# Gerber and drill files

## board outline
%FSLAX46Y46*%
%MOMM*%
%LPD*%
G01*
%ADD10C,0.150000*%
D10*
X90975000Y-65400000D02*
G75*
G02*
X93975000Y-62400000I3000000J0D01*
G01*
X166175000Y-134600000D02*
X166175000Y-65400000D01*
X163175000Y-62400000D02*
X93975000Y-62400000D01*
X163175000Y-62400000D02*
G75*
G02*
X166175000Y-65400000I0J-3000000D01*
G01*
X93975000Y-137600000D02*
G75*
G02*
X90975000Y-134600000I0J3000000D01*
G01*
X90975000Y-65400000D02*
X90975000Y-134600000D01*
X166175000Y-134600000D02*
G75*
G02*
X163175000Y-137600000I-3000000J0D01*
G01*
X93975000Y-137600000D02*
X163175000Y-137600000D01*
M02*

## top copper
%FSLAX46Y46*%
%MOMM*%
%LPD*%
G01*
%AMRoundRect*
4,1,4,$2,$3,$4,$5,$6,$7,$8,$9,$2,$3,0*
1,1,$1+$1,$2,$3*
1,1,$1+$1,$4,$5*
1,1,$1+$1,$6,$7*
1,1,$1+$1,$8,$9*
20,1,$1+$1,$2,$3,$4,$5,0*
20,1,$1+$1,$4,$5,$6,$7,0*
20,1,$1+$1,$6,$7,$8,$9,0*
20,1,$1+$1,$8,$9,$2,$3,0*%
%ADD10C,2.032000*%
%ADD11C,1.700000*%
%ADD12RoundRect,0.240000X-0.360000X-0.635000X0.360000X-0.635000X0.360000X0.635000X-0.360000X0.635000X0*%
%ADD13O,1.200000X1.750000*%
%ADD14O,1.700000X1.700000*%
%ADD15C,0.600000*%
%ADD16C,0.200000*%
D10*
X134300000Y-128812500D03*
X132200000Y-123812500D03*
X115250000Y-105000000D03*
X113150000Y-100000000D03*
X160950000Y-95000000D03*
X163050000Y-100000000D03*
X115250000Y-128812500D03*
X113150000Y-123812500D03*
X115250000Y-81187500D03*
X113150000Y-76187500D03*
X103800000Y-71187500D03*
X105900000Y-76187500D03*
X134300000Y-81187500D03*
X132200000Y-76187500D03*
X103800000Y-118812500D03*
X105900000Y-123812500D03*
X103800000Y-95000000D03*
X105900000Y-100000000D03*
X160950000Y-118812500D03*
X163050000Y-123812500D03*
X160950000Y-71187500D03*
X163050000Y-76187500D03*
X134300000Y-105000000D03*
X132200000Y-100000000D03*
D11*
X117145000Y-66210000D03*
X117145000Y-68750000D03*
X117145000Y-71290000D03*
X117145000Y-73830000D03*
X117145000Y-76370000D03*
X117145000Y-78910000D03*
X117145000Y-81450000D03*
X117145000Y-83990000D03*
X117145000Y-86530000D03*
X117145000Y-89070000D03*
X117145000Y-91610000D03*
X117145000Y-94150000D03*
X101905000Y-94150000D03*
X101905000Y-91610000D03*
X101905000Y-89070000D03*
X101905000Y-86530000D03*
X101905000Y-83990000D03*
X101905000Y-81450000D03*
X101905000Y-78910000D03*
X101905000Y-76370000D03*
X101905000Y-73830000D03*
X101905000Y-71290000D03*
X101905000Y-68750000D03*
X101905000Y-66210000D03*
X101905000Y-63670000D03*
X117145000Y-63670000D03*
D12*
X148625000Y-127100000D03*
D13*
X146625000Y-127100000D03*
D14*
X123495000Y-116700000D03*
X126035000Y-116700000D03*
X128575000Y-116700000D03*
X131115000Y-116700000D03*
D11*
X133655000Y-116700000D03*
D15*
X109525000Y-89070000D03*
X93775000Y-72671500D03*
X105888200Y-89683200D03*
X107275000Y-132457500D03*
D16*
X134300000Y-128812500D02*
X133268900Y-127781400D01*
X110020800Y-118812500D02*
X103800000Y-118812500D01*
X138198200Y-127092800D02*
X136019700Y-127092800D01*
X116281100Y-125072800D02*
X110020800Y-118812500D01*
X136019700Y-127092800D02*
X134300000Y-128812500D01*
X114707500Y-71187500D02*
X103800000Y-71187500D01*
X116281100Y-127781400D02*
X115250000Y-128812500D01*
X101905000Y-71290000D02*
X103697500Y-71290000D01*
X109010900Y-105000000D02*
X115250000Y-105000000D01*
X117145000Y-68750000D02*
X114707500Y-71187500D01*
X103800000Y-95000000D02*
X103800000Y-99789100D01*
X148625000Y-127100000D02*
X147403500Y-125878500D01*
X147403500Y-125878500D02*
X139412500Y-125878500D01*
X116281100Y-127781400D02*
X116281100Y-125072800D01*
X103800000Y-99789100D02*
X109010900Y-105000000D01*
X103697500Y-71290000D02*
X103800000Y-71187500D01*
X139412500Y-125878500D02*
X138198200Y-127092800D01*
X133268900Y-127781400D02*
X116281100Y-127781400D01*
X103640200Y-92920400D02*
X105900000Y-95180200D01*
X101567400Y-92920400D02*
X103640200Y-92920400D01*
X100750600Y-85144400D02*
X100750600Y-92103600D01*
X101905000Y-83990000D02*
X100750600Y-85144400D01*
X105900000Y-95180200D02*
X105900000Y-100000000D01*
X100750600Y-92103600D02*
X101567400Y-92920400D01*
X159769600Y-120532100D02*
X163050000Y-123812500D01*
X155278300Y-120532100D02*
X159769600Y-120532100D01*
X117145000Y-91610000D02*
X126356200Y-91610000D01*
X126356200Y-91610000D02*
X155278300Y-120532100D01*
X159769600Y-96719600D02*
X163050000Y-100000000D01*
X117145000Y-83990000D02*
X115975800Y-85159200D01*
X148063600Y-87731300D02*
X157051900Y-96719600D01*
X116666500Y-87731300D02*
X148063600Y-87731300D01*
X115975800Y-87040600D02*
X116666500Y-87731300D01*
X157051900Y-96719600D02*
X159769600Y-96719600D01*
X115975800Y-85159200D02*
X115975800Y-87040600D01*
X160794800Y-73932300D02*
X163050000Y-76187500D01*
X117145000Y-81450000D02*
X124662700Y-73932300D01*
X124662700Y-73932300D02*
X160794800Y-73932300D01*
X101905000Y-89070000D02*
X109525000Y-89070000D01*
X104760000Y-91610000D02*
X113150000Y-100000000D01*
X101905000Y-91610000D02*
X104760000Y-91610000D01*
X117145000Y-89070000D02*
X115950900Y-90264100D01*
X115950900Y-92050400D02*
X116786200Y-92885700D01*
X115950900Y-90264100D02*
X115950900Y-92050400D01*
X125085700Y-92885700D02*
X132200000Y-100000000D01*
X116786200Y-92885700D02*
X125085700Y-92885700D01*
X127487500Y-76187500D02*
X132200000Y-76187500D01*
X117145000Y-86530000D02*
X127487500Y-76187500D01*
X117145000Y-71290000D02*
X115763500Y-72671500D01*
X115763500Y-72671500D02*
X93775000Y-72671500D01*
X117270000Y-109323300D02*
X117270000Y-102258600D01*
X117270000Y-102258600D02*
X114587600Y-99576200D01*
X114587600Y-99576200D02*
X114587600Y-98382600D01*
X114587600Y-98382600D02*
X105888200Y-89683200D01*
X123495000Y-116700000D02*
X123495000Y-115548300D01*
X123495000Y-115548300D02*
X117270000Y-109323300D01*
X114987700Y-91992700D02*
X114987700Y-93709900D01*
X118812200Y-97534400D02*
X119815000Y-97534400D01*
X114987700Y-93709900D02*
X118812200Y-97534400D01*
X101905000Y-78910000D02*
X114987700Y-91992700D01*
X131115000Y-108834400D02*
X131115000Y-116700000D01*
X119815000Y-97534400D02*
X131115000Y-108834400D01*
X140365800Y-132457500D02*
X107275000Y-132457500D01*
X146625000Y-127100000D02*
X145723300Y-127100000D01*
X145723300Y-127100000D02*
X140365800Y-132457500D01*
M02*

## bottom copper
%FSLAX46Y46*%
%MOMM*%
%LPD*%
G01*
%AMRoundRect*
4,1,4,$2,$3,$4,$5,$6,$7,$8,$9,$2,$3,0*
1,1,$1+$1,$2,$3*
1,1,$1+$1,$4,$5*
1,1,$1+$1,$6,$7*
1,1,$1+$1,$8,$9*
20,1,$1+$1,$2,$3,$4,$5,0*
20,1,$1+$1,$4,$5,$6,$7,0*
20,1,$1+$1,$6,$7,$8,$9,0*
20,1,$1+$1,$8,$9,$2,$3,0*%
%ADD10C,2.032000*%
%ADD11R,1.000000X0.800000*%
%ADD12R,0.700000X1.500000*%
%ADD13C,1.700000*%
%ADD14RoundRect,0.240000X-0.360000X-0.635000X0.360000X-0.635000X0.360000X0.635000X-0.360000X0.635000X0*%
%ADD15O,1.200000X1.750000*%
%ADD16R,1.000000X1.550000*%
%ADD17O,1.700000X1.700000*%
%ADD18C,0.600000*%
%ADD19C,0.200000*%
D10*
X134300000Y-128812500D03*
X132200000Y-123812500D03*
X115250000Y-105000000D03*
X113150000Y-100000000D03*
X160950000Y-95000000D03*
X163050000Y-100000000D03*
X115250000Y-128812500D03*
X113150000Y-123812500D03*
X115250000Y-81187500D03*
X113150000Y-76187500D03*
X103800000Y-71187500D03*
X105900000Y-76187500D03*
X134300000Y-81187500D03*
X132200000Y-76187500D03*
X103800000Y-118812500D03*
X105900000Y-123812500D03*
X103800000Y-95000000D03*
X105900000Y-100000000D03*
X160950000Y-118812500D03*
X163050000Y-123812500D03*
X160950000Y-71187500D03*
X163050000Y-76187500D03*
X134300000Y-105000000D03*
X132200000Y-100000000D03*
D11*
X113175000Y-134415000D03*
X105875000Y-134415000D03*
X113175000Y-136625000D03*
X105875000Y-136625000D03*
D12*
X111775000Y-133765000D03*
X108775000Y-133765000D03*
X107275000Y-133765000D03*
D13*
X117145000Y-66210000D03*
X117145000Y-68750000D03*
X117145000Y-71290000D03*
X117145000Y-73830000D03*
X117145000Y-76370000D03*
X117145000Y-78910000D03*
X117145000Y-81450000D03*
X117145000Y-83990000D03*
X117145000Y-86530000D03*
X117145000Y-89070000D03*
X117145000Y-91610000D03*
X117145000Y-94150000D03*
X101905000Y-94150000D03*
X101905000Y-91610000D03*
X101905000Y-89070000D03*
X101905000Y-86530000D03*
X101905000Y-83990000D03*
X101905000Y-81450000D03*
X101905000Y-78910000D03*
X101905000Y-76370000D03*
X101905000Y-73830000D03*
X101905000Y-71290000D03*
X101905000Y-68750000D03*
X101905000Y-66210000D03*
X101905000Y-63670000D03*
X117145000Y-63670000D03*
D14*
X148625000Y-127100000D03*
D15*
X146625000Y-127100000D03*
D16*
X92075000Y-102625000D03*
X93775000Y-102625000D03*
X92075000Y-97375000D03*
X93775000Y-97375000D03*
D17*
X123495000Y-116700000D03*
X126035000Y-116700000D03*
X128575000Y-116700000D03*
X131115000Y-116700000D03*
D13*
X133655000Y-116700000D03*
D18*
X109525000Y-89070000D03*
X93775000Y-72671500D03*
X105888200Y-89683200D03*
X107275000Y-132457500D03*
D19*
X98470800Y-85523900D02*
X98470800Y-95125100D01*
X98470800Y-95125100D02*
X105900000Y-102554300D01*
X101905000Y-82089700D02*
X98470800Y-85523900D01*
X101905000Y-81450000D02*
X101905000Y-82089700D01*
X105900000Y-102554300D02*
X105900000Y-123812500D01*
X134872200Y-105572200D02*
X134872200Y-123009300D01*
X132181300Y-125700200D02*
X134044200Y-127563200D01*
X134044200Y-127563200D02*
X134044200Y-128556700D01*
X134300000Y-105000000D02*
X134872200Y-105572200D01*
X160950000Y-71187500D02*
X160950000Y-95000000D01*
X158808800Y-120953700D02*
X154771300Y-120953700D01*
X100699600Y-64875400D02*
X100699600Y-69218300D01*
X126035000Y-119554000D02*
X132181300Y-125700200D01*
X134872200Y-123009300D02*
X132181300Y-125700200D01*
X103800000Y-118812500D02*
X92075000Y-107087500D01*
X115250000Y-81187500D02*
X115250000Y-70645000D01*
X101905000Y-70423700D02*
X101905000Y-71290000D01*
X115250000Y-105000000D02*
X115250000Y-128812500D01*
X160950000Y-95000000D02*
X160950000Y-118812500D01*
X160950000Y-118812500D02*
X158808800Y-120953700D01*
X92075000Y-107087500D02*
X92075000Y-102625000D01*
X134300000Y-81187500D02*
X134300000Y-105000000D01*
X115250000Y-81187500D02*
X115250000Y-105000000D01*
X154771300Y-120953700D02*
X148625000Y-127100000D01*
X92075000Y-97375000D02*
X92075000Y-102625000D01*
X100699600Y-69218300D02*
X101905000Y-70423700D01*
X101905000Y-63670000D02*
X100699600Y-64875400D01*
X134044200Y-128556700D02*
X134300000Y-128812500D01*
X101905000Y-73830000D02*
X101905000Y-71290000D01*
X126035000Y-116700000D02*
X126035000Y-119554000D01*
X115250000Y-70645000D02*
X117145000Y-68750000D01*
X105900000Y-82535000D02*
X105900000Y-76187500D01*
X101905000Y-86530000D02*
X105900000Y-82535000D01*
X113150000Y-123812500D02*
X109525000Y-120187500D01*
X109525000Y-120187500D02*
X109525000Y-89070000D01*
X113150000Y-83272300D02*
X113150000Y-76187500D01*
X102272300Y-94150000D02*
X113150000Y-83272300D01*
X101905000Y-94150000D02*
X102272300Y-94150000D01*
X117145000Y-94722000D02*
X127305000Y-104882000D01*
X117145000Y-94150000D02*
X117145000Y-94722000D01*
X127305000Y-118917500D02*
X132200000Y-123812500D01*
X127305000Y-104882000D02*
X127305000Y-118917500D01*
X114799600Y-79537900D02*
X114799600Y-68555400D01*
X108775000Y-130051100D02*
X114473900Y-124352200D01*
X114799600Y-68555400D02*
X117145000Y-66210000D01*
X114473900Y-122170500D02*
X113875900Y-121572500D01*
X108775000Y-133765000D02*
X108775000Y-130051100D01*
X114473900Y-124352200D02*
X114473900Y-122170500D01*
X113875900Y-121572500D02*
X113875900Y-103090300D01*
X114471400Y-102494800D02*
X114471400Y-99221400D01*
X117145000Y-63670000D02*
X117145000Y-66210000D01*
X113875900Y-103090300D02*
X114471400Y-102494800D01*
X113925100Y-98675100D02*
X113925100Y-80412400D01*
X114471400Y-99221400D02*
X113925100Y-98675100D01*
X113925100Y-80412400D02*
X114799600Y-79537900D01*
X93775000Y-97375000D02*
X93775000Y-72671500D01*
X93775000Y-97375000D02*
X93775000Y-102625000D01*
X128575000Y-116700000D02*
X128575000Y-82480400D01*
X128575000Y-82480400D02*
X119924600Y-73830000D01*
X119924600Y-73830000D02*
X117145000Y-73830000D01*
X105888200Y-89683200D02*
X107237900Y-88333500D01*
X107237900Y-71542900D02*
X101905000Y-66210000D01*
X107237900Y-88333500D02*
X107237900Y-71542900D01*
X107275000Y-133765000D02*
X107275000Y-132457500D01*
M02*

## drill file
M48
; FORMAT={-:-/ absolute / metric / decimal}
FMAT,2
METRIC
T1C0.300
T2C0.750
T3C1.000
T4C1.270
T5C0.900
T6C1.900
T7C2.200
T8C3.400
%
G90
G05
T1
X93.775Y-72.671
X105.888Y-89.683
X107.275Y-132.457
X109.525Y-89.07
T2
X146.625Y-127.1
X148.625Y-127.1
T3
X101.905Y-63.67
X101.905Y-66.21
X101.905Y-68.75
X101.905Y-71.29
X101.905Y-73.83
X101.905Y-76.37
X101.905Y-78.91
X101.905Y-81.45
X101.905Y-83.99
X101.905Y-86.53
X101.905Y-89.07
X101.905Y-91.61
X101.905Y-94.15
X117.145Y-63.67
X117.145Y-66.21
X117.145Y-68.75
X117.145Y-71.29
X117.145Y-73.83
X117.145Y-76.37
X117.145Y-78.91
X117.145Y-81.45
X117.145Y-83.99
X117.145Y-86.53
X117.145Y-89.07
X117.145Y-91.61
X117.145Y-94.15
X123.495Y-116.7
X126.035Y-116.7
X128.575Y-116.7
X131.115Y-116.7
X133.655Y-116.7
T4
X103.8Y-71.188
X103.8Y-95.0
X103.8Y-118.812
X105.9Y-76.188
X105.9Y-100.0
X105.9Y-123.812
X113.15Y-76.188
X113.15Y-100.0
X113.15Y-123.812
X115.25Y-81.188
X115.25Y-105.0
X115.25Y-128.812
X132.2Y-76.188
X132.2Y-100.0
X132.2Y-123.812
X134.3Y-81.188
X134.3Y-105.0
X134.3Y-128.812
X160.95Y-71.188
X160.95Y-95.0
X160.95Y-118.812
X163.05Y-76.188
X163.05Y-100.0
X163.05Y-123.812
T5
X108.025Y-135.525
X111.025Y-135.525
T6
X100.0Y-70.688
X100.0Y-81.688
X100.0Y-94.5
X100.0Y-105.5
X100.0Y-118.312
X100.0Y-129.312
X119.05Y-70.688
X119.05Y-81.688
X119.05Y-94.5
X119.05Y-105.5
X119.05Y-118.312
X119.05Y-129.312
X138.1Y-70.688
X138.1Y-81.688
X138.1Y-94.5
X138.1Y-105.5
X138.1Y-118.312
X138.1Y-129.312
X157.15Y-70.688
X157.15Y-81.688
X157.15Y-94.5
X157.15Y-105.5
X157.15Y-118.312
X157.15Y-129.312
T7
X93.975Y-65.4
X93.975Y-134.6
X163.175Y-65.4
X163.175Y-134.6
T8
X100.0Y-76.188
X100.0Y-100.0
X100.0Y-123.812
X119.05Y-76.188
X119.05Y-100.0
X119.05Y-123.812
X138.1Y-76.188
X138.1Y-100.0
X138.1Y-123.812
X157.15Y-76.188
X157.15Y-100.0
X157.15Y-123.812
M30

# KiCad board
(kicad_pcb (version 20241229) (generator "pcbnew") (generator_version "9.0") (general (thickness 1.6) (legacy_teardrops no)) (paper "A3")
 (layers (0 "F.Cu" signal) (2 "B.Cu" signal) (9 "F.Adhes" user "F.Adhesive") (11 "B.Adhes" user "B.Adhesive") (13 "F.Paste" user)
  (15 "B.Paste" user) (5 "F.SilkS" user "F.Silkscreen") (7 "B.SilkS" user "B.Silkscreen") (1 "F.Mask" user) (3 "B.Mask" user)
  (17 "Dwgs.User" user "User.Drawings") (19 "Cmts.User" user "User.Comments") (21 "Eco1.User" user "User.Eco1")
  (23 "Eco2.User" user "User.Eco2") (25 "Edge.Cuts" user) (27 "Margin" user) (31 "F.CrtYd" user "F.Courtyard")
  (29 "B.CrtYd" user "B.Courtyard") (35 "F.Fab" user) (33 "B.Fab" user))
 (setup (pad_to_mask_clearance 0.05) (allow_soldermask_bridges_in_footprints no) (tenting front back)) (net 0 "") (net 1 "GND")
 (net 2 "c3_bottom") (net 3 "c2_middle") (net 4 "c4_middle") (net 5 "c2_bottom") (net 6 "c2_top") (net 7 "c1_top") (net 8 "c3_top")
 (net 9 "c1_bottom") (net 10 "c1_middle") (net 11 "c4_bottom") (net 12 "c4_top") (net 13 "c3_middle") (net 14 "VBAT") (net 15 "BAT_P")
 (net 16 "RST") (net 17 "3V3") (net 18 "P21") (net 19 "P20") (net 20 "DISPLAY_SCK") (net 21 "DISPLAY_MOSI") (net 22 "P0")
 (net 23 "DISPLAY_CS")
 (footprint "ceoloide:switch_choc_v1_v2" (layer "F.Cu") (at 138.1 123.8125 90)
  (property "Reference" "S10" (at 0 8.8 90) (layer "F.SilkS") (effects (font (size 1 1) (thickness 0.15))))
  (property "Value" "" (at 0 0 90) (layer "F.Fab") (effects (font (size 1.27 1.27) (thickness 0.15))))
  (pad "" np_thru_hole circle (at -5.5 0 90) (size 1.9 1.9) (drill 1.9) (layers "*.Cu" "*.Mask"))
  (pad "" np_thru_hole circle (at 0 0 90) (size 3.4 3.4) (drill 3.4) (layers "*.Cu" "*.Mask"))
  (pad "" np_thru_hole circle (at 5.5 0 90) (size 1.9 1.9) (drill 1.9) (layers "*.Cu" "*.Mask"))
  (pad "1" thru_hole circle (at -5 -3.8 285) (size 2.032 2.032) (drill 1.27) (layers "*.Cu" "*.Mask") (remove_unused_layers no)
   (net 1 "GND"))
  (pad "2" thru_hole circle (at 0 -5.9 285) (size 2.032 2.032) (drill 1.27) (layers "*.Cu" "*.Mask") (remove_unused_layers no)
   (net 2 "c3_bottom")))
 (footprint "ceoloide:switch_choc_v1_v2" (layer "F.Cu") (at 119.05 100 90)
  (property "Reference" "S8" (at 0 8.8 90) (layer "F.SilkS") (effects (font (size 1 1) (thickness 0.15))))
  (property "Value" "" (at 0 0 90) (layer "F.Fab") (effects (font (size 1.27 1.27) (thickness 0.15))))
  (pad "" np_thru_hole circle (at -5.5 0 90) (size 1.9 1.9) (drill 1.9) (layers "*.Cu" "*.Mask"))
  (pad "" np_thru_hole circle (at 0 0 90) (size 3.4 3.4) (drill 3.4) (layers "*.Cu" "*.Mask"))
  (pad "" np_thru_hole circle (at 5.5 0 90) (size 1.9 1.9) (drill 1.9) (layers "*.Cu" "*.Mask"))
  (pad "1" thru_hole circle (at -5 -3.8 285) (size 2.032 2.032) (drill 1.27) (layers "*.Cu" "*.Mask") (remove_unused_layers no)
   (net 1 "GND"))
  (pad "2" thru_hole circle (at 0 -5.9 285) (size 2.032 2.032) (drill 1.27) (layers "*.Cu" "*.Mask") (remove_unused_layers no)
   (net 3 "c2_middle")))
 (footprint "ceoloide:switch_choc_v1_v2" (layer "F.Cu") (at 157.15 100 -90)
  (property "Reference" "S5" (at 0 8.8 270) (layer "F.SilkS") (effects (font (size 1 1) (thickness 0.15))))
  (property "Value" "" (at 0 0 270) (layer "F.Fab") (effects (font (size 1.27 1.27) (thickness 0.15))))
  (pad "" np_thru_hole circle (at -5.5 0 270) (size 1.9 1.9) (drill 1.9) (layers "*.Cu" "*.Mask"))
  (pad "" np_thru_hole circle (at 0 0 270) (size 3.4 3.4) (drill 3.4) (layers "*.Cu" "*.Mask"))
  (pad "" np_thru_hole circle (at 5.5 0 270) (size 1.9 1.9) (drill 1.9) (layers "*.Cu" "*.Mask"))
  (pad "1" thru_hole circle (at -5 -3.8 105) (size 2.032 2.032) (drill 1.27) (layers "*.Cu" "*.Mask") (remove_unused_layers no)
   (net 1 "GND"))
  (pad "2" thru_hole circle (at 0 -5.9 105) (size 2.032 2.032) (drill 1.27) (layers "*.Cu" "*.Mask") (remove_unused_layers no)
   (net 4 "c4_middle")))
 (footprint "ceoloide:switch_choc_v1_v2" (layer "F.Cu") (at 119.05 123.8125 90)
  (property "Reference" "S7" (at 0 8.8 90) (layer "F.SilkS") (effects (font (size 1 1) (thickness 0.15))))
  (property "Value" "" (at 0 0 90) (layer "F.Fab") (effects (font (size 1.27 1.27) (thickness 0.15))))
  (pad "" np_thru_hole circle (at -5.5 0 90) (size 1.9 1.9) (drill 1.9) (layers "*.Cu" "*.Mask"))
  (pad "" np_thru_hole circle (at 0 0 90) (size 3.4 3.4) (drill 3.4) (layers "*.Cu" "*.Mask"))
  (pad "" np_thru_hole circle (at 5.5 0 90) (size 1.9 1.9) (drill 1.9) (layers "*.Cu" "*.Mask"))
  (pad "1" thru_hole circle (at -5 -3.8 285) (size 2.032 2.032) (drill 1.27) (layers "*.Cu" "*.Mask") (remove_unused_layers no)
   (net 1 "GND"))
  (pad "2" thru_hole circle (at 0 -5.9 285) (size 2.032 2.032) (drill 1.27) (layers "*.Cu" "*.Mask") (remove_unused_layers no)
   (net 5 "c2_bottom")))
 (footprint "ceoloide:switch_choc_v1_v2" (layer "F.Cu") (at 119.05 76.1875 90)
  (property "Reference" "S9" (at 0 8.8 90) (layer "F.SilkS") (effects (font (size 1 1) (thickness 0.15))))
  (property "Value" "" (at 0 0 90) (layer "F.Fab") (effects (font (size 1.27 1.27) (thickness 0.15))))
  (pad "" np_thru_hole circle (at -5.5 0 90) (size 1.9 1.9) (drill 1.9) (layers "*.Cu" "*.Mask"))
  (pad "" np_thru_hole circle (at 0 0 90) (size 3.4 3.4) (drill 3.4) (layers "*.Cu" "*.Mask"))
  (pad "" np_thru_hole circle (at 5.5 0 90) (size 1.9 1.9) (drill 1.9) (layers "*.Cu" "*.Mask"))
  (pad "1" thru_hole circle (at -5 -3.8 285) (size 2.032 2.032) (drill 1.27) (layers "*.Cu" "*.Mask") (remove_unused_layers no)
   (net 1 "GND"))
  (pad "2" thru_hole circle (at 0 -5.9 285) (size 2.032 2.032) (drill 1.27) (layers "*.Cu" "*.Mask") (remove_unused_layers no)
   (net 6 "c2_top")))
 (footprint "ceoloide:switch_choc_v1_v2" (layer "F.Cu") (at 100 76.1875 -90)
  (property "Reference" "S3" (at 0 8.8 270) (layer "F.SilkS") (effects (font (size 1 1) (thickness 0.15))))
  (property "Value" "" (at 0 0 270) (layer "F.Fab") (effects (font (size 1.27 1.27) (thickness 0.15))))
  (pad "" np_thru_hole circle (at -5.5 0 270) (size 1.9 1.9) (drill 1.9) (layers "*.Cu" "*.Mask"))
  (pad "" np_thru_hole circle (at 0 0 270) (size 3.4 3.4) (drill 3.4) (layers "*.Cu" "*.Mask"))
  (pad "" np_thru_hole circle (at 5.5 0 270) (size 1.9 1.9) (drill 1.9) (layers "*.Cu" "*.Mask"))
  (pad "1" thru_hole circle (at -5 -3.8 105) (size 2.032 2.032) (drill 1.27) (layers "*.Cu" "*.Mask") (remove_unused_layers no)
   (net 1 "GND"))
  (pad "2" thru_hole circle (at 0 -5.9 105) (size 2.032 2.032) (drill 1.27) (layers "*.Cu" "*.Mask") (remove_unused_layers no)
   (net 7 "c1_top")))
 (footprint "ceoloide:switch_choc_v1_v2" (layer "F.Cu") (at 138.1 76.1875 90)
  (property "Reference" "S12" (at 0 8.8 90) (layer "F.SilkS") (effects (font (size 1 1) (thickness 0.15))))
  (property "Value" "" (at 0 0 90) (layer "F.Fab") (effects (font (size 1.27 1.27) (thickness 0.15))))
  (pad "" np_thru_hole circle (at -5.5 0 90) (size 1.9 1.9) (drill 1.9) (layers "*.Cu" "*.Mask"))
  (pad "" np_thru_hole circle (at 0 0 90) (size 3.4 3.4) (drill 3.4) (layers "*.Cu" "*.Mask"))
  (pad "" np_thru_hole circle (at 5.5 0 90) (size 1.9 1.9) (drill 1.9) (layers "*.Cu" "*.Mask"))
  (pad "1" thru_hole circle (at -5 -3.8 285) (size 2.032 2.032) (drill 1.27) (layers "*.Cu" "*.Mask") (remove_unused_layers no)
   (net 1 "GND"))
  (pad "2" thru_hole circle (at 0 -5.9 285) (size 2.032 2.032) (drill 1.27) (layers "*.Cu" "*.Mask") (remove_unused_layers no)
   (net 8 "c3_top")))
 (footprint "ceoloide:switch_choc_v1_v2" (layer "F.Cu") (at 100 123.8125 -90)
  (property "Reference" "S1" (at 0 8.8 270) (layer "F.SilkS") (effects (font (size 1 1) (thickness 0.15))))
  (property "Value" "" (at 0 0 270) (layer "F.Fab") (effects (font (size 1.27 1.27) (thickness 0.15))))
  (pad "" np_thru_hole circle (at -5.5 0 270) (size 1.9 1.9) (drill 1.9) (layers "*.Cu" "*.Mask"))
  (pad "" np_thru_hole circle (at 0 0 270) (size 3.4 3.4) (drill 3.4) (layers "*.Cu" "*.Mask"))
  (pad "" np_thru_hole circle (at 5.5 0 270) (size 1.9 1.9) (drill 1.9) (layers "*.Cu" "*.Mask"))
  (pad "1" thru_hole circle (at -5 -3.8 105) (size 2.032 2.032) (drill 1.27) (layers "*.Cu" "*.Mask") (remove_unused_layers no)
   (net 1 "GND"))
  (pad "2" thru_hole circle (at 0 -5.9 105) (size 2.032 2.032) (drill 1.27) (layers "*.Cu" "*.Mask") (remove_unused_layers no)
   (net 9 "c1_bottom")))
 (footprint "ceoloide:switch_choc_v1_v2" (layer "F.Cu") (at 100 100 -90)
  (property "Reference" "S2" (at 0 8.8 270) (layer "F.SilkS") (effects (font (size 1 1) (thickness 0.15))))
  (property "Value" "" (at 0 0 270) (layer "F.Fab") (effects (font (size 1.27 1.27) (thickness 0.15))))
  (pad "" np_thru_hole circle (at -5.5 0 270) (size 1.9 1.9) (drill 1.9) (layers "*.Cu" "*.Mask"))
  (pad "" np_thru_hole circle (at 0 0 270) (size 3.4 3.4) (drill 3.4) (layers "*.Cu" "*.Mask"))
  (pad "" np_thru_hole circle (at 5.5 0 270) (size 1.9 1.9) (drill 1.9) (layers "*.Cu" "*.Mask"))
  (pad "1" thru_hole circle (at -5 -3.8 105) (size 2.032 2.032) (drill 1.27) (layers "*.Cu" "*.Mask") (remove_unused_layers no)
   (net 1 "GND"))
  (pad "2" thru_hole circle (at 0 -5.9 105) (size 2.032 2.032) (drill 1.27) (layers "*.Cu" "*.Mask") (remove_unused_layers no)
   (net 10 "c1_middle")))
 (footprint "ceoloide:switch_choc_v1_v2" (layer "F.Cu") (at 157.15 123.8125 -90)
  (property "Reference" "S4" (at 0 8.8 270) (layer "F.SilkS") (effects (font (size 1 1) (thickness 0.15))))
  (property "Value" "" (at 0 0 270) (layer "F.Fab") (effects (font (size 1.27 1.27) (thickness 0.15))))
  (pad "" np_thru_hole circle (at -5.5 0 270) (size 1.9 1.9) (drill 1.9) (layers "*.Cu" "*.Mask"))
  (pad "" np_thru_hole circle (at 0 0 270) (size 3.4 3.4) (drill 3.4) (layers "*.Cu" "*.Mask"))
  (pad "" np_thru_hole circle (at 5.5 0 270) (size 1.9 1.9) (drill 1.9) (layers "*.Cu" "*.Mask"))
  (pad "1" thru_hole circle (at -5 -3.8 105) (size 2.032 2.032) (drill 1.27) (layers "*.Cu" "*.Mask") (remove_unused_layers no)
   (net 1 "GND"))
  (pad "2" thru_hole circle (at 0 -5.9 105) (size 2.032 2.032) (drill 1.27) (layers "*.Cu" "*.Mask") (remove_unused_layers no)
   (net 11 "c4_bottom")))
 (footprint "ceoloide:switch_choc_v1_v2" (layer "F.Cu") (at 157.15 76.1875 -90)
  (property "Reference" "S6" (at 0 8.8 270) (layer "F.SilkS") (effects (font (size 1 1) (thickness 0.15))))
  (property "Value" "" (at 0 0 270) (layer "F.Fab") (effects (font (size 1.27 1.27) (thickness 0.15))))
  (pad "" np_thru_hole circle (at -5.5 0 270) (size 1.9 1.9) (drill 1.9) (layers "*.Cu" "*.Mask"))
  (pad "" np_thru_hole circle (at 0 0 270) (size 3.4 3.4) (drill 3.4) (layers "*.Cu" "*.Mask"))
  (pad "" np_thru_hole circle (at 5.5 0 270) (size 1.9 1.9) (drill 1.9) (layers "*.Cu" "*.Mask"))
  (pad "1" thru_hole circle (at -5 -3.8 105) (size 2.032 2.032) (drill 1.27) (layers "*.Cu" "*.Mask") (remove_unused_layers no)
   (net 1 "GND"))
  (pad "2" thru_hole circle (at 0 -5.9 105) (size 2.032 2.032) (drill 1.27) (layers "*.Cu" "*.Mask") (remove_unused_layers no)
   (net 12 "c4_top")))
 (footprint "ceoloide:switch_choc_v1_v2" (layer "F.Cu") (at 138.1 100 90)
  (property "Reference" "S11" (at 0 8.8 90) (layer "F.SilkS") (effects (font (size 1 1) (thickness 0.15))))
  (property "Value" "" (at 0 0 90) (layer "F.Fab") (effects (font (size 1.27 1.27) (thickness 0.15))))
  (pad "" np_thru_hole circle (at -5.5 0 90) (size 1.9 1.9) (drill 1.9) (layers "*.Cu" "*.Mask"))
  (pad "" np_thru_hole circle (at 0 0 90) (size 3.4 3.4) (drill 3.4) (layers "*.Cu" "*.Mask"))
  (pad "" np_thru_hole circle (at 5.5 0 90) (size 1.9 1.9) (drill 1.9) (layers "*.Cu" "*.Mask"))
  (pad "1" thru_hole circle (at -5 -3.8 285) (size 2.032 2.032) (drill 1.27) (layers "*.Cu" "*.Mask") (remove_unused_layers no)
   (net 1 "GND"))
  (pad "2" thru_hole circle (at 0 -5.9 285) (size 2.032 2.032) (drill 1.27) (layers "*.Cu" "*.Mask") (remove_unused_layers no)
   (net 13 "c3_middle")))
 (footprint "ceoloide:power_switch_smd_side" (layer "B.Cu") (at 109.525 135.5 -90)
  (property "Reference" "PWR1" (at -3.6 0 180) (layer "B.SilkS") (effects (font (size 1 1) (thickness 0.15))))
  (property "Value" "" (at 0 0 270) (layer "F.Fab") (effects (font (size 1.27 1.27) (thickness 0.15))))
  (pad "" smd rect (at -1.085 -3.65 180) (size 1 0.8) (layers "B.Cu" "B.Mask" "B.Paste"))
  (pad "" smd rect (at -1.085 3.65 180) (size 1 0.8) (layers "B.Cu" "B.Mask" "B.Paste"))
  (pad "" np_thru_hole circle (at 0.025 -1.5) (size 0.9 0.9) (drill 0.9) (layers "*.Cu" "*.Mask"))
  (pad "" np_thru_hole circle (at 0.025 1.5) (size 0.9 0.9) (drill 0.9) (layers "*.Cu" "*.Mask"))
  (pad "" smd rect (at 1.125 -3.65 180) (size 1 0.8) (layers "B.Cu" "B.Mask" "B.Paste"))
  (pad "" smd rect (at 1.125 3.65 180) (size 1 0.8) (layers "B.Cu" "B.Mask" "B.Paste"))
  (pad "1" smd rect (at -1.735 -2.25 180) (size 0.7 1.5) (layers "B.Cu" "B.Mask" "B.Paste"))
  (pad "2" smd rect (at -1.735 0.75 180) (size 0.7 1.5) (layers "B.Cu" "B.Mask" "B.Paste") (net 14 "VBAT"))
  (pad "3" smd rect (at -1.735 2.25 180) (size 0.7 1.5) (layers "B.Cu" "B.Mask" "B.Paste") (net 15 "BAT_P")))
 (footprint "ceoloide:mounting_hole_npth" (layer "B.Cu") (at 93.975 134.6)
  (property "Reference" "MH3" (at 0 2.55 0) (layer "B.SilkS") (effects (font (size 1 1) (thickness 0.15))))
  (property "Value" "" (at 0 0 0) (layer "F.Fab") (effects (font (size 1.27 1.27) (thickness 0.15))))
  (pad "" np_thru_hole circle (at 0 0) (size 2.2 2.2) (drill 2.2) (layers "*.Cu" "*.Mask")))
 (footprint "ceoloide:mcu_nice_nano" (layer "B.Cu") (at 109.525 78.91)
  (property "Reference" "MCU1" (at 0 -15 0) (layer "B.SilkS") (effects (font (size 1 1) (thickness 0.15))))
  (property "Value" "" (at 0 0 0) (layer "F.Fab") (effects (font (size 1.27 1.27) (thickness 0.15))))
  (pad "1" thru_hole circle (at 7.62 -12.7) (size 1.7 1.7) (drill 1) (layers "*.Cu" "*.Mask") (remove_unused_layers no) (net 14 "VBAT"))
  (pad "2" thru_hole circle (at 7.62 -10.16) (size 1.7 1.7) (drill 1) (layers "*.Cu" "*.Mask") (remove_unused_layers no) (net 1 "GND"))
  (pad "3" thru_hole circle (at 7.62 -7.62) (size 1.7 1.7) (drill 1) (layers "*.Cu" "*.Mask") (remove_unused_layers no) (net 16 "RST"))
  (pad "4" thru_hole circle (at 7.62 -5.08) (size 1.7 1.7) (drill 1) (layers "*.Cu" "*.Mask") (remove_unused_layers no) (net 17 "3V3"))
  (pad "5" thru_hole circle (at 7.62 -2.54) (size 1.7 1.7) (drill 1) (layers "*.Cu" "*.Mask") (remove_unused_layers no) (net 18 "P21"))
  (pad "6" thru_hole circle (at 7.62 0) (size 1.7 1.7) (drill 1) (layers "*.Cu" "*.Mask") (remove_unused_layers no) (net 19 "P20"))
  (pad "7" thru_hole circle (at 7.62 2.54) (size 1.7 1.7) (drill 1) (layers "*.Cu" "*.Mask") (remove_unused_layers no) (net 12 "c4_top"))
  (pad "8" thru_hole circle (at 7.62 5.08) (size 1.7 1.7) (drill 1) (layers "*.Cu" "*.Mask") (remove_unused_layers no) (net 4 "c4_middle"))
  (pad "9" thru_hole circle (at 7.62 7.62) (size 1.7 1.7) (drill 1) (layers "*.Cu" "*.Mask") (remove_unused_layers no) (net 8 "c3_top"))
  (pad "10" thru_hole circle (at 7.62 10.16) (size 1.7 1.7) (drill 1) (layers "*.Cu" "*.Mask") (remove_unused_layers no)
   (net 13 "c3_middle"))
  (pad "11" thru_hole circle (at 7.62 12.7) (size 1.7 1.7) (drill 1) (layers "*.Cu" "*.Mask") (remove_unused_layers no) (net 11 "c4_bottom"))
  (pad "12" thru_hole circle (at 7.62 15.24) (size 1.7 1.7) (drill 1) (layers "*.Cu" "*.Mask") (remove_unused_layers no) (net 2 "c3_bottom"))
  (pad "13" thru_hole circle (at -7.62 15.24) (size 1.7 1.7) (drill 1) (layers "*.Cu" "*.Mask") (remove_unused_layers no) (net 6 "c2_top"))
  (pad "14" thru_hole circle (at -7.62 12.7) (size 1.7 1.7) (drill 1) (layers "*.Cu" "*.Mask") (remove_unused_layers no) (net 3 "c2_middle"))
  (pad "15" thru_hole circle (at -7.62 10.16) (size 1.7 1.7) (drill 1) (layers "*.Cu" "*.Mask") (remove_unused_layers no)
   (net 5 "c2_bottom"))
  (pad "16" thru_hole circle (at -7.62 7.62) (size 1.7 1.7) (drill 1) (layers "*.Cu" "*.Mask") (remove_unused_layers no) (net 7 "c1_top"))
  (pad "17" thru_hole circle (at -7.62 5.08) (size 1.7 1.7) (drill 1) (layers "*.Cu" "*.Mask") (remove_unused_layers no)
   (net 10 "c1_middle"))
  (pad "18" thru_hole circle (at -7.62 2.54) (size 1.7 1.7) (drill 1) (layers "*.Cu" "*.Mask") (remove_unused_layers no) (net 9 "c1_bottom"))
  (pad "19" thru_hole circle (at -7.62 0) (size 1.7 1.7) (drill 1) (layers "*.Cu" "*.Mask") (remove_unused_layers no) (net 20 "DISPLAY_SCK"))
  (pad "20" thru_hole circle (at -7.62 -2.54) (size 1.7 1.7) (drill 1) (layers "*.Cu" "*.Mask") (remove_unused_layers no)
   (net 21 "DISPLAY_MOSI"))
  (pad "21" thru_hole circle (at -7.62 -5.08) (size 1.7 1.7) (drill 1) (layers "*.Cu" "*.Mask") (remove_unused_layers no) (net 1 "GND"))
  (pad "22" thru_hole circle (at -7.62 -7.62) (size 1.7 1.7) (drill 1) (layers "*.Cu" "*.Mask") (remove_unused_layers no) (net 1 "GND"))
  (pad "23" thru_hole circle (at -7.62 -10.16) (size 1.7 1.7) (drill 1) (layers "*.Cu" "*.Mask") (remove_unused_layers no) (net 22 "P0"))
  (pad "24" thru_hole circle (at -7.62 -12.7) (size 1.7 1.7) (drill 1) (layers "*.Cu" "*.Mask") (remove_unused_layers no)
   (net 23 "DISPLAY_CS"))
  (pad "25" thru_hole circle (at -7.62 -15.24) (size 1.7 1.7) (drill 1) (layers "*.Cu" "*.Mask") (remove_unused_layers no) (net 1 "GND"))
  (pad "26" thru_hole circle (at 7.62 -15.24) (size 1.7 1.7) (drill 1) (layers "*.Cu" "*.Mask") (remove_unused_layers no) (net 14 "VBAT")))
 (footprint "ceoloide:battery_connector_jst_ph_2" (layer "B.Cu") (at 147.625 127.1)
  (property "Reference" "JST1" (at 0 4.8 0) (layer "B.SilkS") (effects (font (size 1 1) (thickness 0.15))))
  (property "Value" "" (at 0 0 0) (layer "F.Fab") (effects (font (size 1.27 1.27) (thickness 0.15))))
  (pad "1" thru_hole roundrect (at 1 0) (size 1.2 1.75) (drill 0.75) (layers "*.Cu" "*.Mask") (remove_unused_layers no)
   (roundrect_rratio 0.2) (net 1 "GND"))
  (pad "2" thru_hole oval (at -1 0) (size 1.2 1.75) (drill 0.75) (layers "*.Cu" "*.Mask") (remove_unused_layers no) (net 15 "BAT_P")))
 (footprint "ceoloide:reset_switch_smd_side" (layer "B.Cu") (at 92.925 100 90)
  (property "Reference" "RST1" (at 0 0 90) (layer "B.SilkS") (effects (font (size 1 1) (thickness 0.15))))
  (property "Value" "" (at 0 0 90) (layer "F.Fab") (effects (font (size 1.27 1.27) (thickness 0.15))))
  (pad "1" smd rect (at -2.625 -0.85 270) (size 1.55 1) (layers "B.Cu" "B.Mask" "B.Paste") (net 1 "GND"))
  (pad "2" smd rect (at -2.625 0.85 270) (size 1.55 1) (layers "B.Cu" "B.Mask" "B.Paste") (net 16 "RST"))
  (pad "3" smd rect (at 2.625 -0.85 270) (size 1.55 1) (layers "B.Cu" "B.Mask" "B.Paste") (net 1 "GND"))
  (pad "4" smd rect (at 2.625 0.85 270) (size 1.55 1) (layers "B.Cu" "B.Mask" "B.Paste") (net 16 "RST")))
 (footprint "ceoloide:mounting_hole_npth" (layer "B.Cu") (at 163.175 65.4)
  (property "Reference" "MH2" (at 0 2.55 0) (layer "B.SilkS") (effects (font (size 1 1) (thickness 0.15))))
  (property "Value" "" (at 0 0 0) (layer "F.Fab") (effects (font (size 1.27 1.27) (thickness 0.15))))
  (pad "" np_thru_hole circle (at 0 0) (size 2.2 2.2) (drill 2.2) (layers "*.Cu" "*.Mask")))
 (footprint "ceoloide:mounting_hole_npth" (layer "B.Cu") (at 163.175 134.6)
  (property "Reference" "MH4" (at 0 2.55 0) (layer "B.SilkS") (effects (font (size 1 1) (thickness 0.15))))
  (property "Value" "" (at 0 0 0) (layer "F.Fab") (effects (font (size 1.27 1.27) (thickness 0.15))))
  (pad "" np_thru_hole circle (at 0 0) (size 2.2 2.2) (drill 2.2) (layers "*.Cu" "*.Mask")))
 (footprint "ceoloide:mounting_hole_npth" (layer "B.Cu") (at 93.975 65.4)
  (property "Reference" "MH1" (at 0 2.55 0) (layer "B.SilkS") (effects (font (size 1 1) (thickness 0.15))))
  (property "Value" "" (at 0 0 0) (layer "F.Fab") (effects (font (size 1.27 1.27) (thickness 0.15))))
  (pad "" np_thru_hole circle (at 0 0) (size 2.2 2.2) (drill 2.2) (layers "*.Cu" "*.Mask")))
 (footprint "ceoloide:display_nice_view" (layer "B.Cu") (at 128.575 100)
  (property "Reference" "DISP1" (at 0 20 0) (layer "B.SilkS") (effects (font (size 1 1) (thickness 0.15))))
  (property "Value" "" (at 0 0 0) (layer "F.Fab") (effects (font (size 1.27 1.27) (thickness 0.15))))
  (pad "1" thru_hole oval (at -5.08 16.7 270) (size 1.7 1.7) (drill 1) (layers "*.Cu" "*.Mask") (remove_unused_layers no)
   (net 23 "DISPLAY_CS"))
  (pad "2" thru_hole oval (at -2.54 16.7 270) (size 1.7 1.7) (drill 1) (layers "*.Cu" "*.Mask") (remove_unused_layers no) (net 1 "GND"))
  (pad "3" thru_hole oval (at 0 16.7 270) (size 1.7 1.7) (drill 1) (layers "*.Cu" "*.Mask") (remove_unused_layers no) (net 17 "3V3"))
  (pad "4" thru_hole oval (at 2.54 16.7 270) (size 1.7 1.7) (drill 1) (layers "*.Cu" "*.Mask") (remove_unused_layers no)
   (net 20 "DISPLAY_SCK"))
  (pad "5" thru_hole circle (at 5.08 16.7 270) (size 1.7 1.7) (drill 1) (layers "*.Cu" "*.Mask") (remove_unused_layers no)
   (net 21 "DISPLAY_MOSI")))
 (gr_arc (start 90.975 65.4) (mid 91.85368 63.27868) (end 93.975 62.4) (stroke (width 0.15) (type default)) (layer "Edge.Cuts"))
 (gr_line (start 166.175 134.6) (end 166.175 65.4) (stroke (width 0.15) (type default)) (layer "Edge.Cuts"))
 (gr_line (start 163.175 62.4) (end 93.975 62.4) (stroke (width 0.15) (type default)) (layer "Edge.Cuts"))
 (gr_arc (start 163.175 62.4) (mid 165.29632 63.27868) (end 166.175 65.4) (stroke (width 0.15) (type default)) (layer "Edge.Cuts"))
 (gr_arc (start 93.975 137.6) (mid 91.85368 136.72132) (end 90.975 134.6) (stroke (width 0.15) (type default)) (layer "Edge.Cuts"))
 (gr_line (start 90.975 65.4) (end 90.975 134.6) (stroke (width 0.15) (type default)) (layer "Edge.Cuts"))
 (gr_arc (start 166.175 134.6) (mid 165.29632 136.72132) (end 163.175 137.6) (stroke (width 0.15) (type default)) (layer "Edge.Cuts"))
 (gr_line (start 93.975 137.6) (end 163.175 137.6) (stroke (width 0.15) (type default)) (layer "Edge.Cuts"))
 (segment (start 98.4708 85.5239) (end 98.4708 95.1251) (width 0.2) (layer "B.Cu") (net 9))
 (segment (start 98.4708 95.1251) (end 105.9 102.5543) (width 0.2) (layer "B.Cu") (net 9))
 (segment (start 101.905 82.0897) (end 98.4708 85.5239) (width 0.2) (layer "B.Cu") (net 9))
 (segment (start 101.905 81.45) (end 101.905 82.0897) (width 0.2) (layer "B.Cu") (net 9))
 (segment (start 105.9 102.5543) (end 105.9 123.8125) (width 0.2) (layer "B.Cu") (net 9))
 (segment (start 134.3 128.8125) (end 133.2689 127.7814) (width 0.2) (layer "F.Cu") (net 1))
 (segment (start 110.0208 118.8125) (end 103.8 118.8125) (width 0.2) (layer "F.Cu") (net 1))
 (segment (start 138.1982 127.0928) (end 136.0197 127.0928) (width 0.2) (layer "F.Cu") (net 1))
 (segment (start 116.2811 125.0728) (end 110.0208 118.8125) (width 0.2) (layer "F.Cu") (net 1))
 (segment (start 136.0197 127.0928) (end 134.3 128.8125) (width 0.2) (layer "F.Cu") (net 1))
 (segment (start 114.7075 71.1875) (end 103.8 71.1875) (width 0.2) (layer "F.Cu") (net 1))
 (segment (start 116.2811 127.7814) (end 115.25 128.8125) (width 0.2) (layer "F.Cu") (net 1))
 (segment (start 101.905 71.29) (end 103.6975 71.29) (width 0.2) (layer "F.Cu") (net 1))
 (segment (start 109.0109 105) (end 115.25 105) (width 0.2) (layer "F.Cu") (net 1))
 (segment (start 117.145 68.75) (end 114.7075 71.1875) (width 0.2) (layer "F.Cu") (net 1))
 (segment (start 103.8 95) (end 103.8 99.7891) (width 0.2) (layer "F.Cu") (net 1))
 (segment (start 148.625 127.1) (end 147.4035 125.8785) (width 0.2) (layer "F.Cu") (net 1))
 (segment (start 147.4035 125.8785) (end 139.4125 125.8785) (width 0.2) (layer "F.Cu") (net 1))
 (segment (start 116.2811 127.7814) (end 116.2811 125.0728) (width 0.2) (layer "F.Cu") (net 1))
 (segment (start 103.8 99.7891) (end 109.0109 105) (width 0.2) (layer "F.Cu") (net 1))
 (segment (start 103.6975 71.29) (end 103.8 71.1875) (width 0.2) (layer "F.Cu") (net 1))
 (segment (start 139.4125 125.8785) (end 138.1982 127.0928) (width 0.2) (layer "F.Cu") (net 1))
 (segment (start 133.2689 127.7814) (end 116.2811 127.7814) (width 0.2) (layer "F.Cu") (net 1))
 (segment (start 134.8722 105.5722) (end 134.8722 123.0093) (width 0.2) (layer "B.Cu") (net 1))
 (segment (start 132.1813 125.7002) (end 134.0442 127.5632) (width 0.2) (layer "B.Cu") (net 1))
 (segment (start 134.0442 127.5632) (end 134.0442 128.5567) (width 0.2) (layer "B.Cu") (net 1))
 (segment (start 134.3 105) (end 134.8722 105.5722) (width 0.2) (layer "B.Cu") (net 1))
 (segment (start 160.95 71.1875) (end 160.95 95) (width 0.2) (layer "B.Cu") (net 1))
 (segment (start 158.8088 120.9537) (end 154.7713 120.9537) (width 0.2) (layer "B.Cu") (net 1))
 (segment (start 100.6996 64.8754) (end 100.6996 69.2183) (width 0.2) (layer "B.Cu") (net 1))
 (segment (start 126.035 119.554) (end 132.1813 125.7002) (width 0.2) (layer "B.Cu") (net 1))
 (segment (start 134.8722 123.0093) (end 132.1813 125.7002) (width 0.2) (layer "B.Cu") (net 1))
 (segment (start 103.8 118.8125) (end 92.075 107.0875) (width 0.2) (layer "B.Cu") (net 1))
 (segment (start 115.25 81.1875) (end 115.25 70.645) (width 0.2) (layer "B.Cu") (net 1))
 (segment (start 101.905 70.4237) (end 101.905 71.29) (width 0.2) (layer "B.Cu") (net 1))
 (segment (start 115.25 105) (end 115.25 128.8125) (width 0.2) (layer "B.Cu") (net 1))
 (segment (start 160.95 95) (end 160.95 118.8125) (width 0.2) (layer "B.Cu") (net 1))
 (segment (start 160.95 118.8125) (end 158.8088 120.9537) (width 0.2) (layer "B.Cu") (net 1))
 (segment (start 92.075 107.0875) (end 92.075 102.625) (width 0.2) (layer "B.Cu") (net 1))
 (segment (start 134.3 81.1875) (end 134.3 105) (width 0.2) (layer "B.Cu") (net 1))
 (segment (start 115.25 81.1875) (end 115.25 105) (width 0.2) (layer "B.Cu") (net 1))
 (segment (start 154.7713 120.9537) (end 148.625 127.1) (width 0.2) (layer "B.Cu") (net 1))
 (segment (start 92.075 97.375) (end 92.075 102.625) (width 0.2) (layer "B.Cu") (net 1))
 (segment (start 100.6996 69.2183) (end 101.905 70.4237) (width 0.2) (layer "B.Cu") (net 1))
 (segment (start 101.905 63.67) (end 100.6996 64.8754) (width 0.2) (layer "B.Cu") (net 1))
 (segment (start 134.0442 128.5567) (end 134.3 128.8125) (width 0.2) (layer "B.Cu") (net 1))
 (segment (start 101.905 73.83) (end 101.905 71.29) (width 0.2) (layer "B.Cu") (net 1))
 (segment (start 126.035 116.7) (end 126.035 119.554) (width 0.2) (layer "B.Cu") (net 1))
 (segment (start 115.25 70.645) (end 117.145 68.75) (width 0.2) (layer "B.Cu") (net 1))
 (segment (start 103.6402 92.9204) (end 105.9 95.1802) (width 0.2) (layer "F.Cu") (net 10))
 (segment (start 101.5674 92.9204) (end 103.6402 92.9204) (width 0.2) (layer "F.Cu") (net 10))
 (segment (start 100.7506 85.1444) (end 100.7506 92.1036) (width 0.2) (layer "F.Cu") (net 10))
 (segment (start 101.905 83.99) (end 100.7506 85.1444) (width 0.2) (layer "F.Cu") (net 10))
 (segment (start 105.9 95.1802) (end 105.9 100) (width 0.2) (layer "F.Cu") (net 10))
 (segment (start 100.7506 92.1036) (end 101.5674 92.9204) (width 0.2) (layer "F.Cu") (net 10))
 (segment (start 105.9 82.535) (end 105.9 76.1875) (width 0.2) (layer "B.Cu") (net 7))
 (segment (start 101.905 86.53) (end 105.9 82.535) (width 0.2) (layer "B.Cu") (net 7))
 (segment (start 159.7696 120.5321) (end 163.05 123.8125) (width 0.2) (layer "F.Cu") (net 11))
 (segment (start 155.2783 120.5321) (end 159.7696 120.5321) (width 0.2) (layer "F.Cu") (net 11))
 (segment (start 117.145 91.61) (end 126.3562 91.61) (width 0.2) (layer "F.Cu") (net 11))
 (segment (start 126.3562 91.61) (end 155.2783 120.5321) (width 0.2) (layer "F.Cu") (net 11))
 (segment (start 159.7696 96.7196) (end 163.05 100) (width 0.2) (layer "F.Cu") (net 4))
 (segment (start 117.145 83.99) (end 115.9758 85.1592) (width 0.2) (layer "F.Cu") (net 4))
 (segment (start 148.0636 87.7313) (end 157.0519 96.7196) (width 0.2) (layer "F.Cu") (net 4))
 (segment (start 116.6665 87.7313) (end 148.0636 87.7313) (width 0.2) (layer "F.Cu") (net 4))
 (segment (start 115.9758 87.0406) (end 116.6665 87.7313) (width 0.2) (layer "F.Cu") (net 4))
 (segment (start 157.0519 96.7196) (end 159.7696 96.7196) (width 0.2) (layer "F.Cu") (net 4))
 (segment (start 115.9758 85.1592) (end 115.9758 87.0406) (width 0.2) (layer "F.Cu") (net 4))
 (segment (start 160.7948 73.9323) (end 163.05 76.1875) (width 0.2) (layer "F.Cu") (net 12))
 (segment (start 117.145 81.45) (end 124.6627 73.9323) (width 0.2) (layer "F.Cu") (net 12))
 (segment (start 124.6627 73.9323) (end 160.7948 73.9323) (width 0.2) (layer "F.Cu") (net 12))
 (segment (start 101.905 89.07) (end 109.525 89.07) (width 0.2) (layer "F.Cu") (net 5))
 (via (at 109.525 89.07) (size 0.6) (drill 0.3) (layers "F.Cu" "B.Cu") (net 5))
 (segment (start 113.15 123.8125) (end 109.525 120.1875) (width 0.2) (layer "B.Cu") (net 5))
 (segment (start 109.525 120.1875) (end 109.525 89.07) (width 0.2) (layer "B.Cu") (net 5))
 (segment (start 104.76 91.61) (end 113.15 100) (width 0.2) (layer "F.Cu") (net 3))
 (segment (start 101.905 91.61) (end 104.76 91.61) (width 0.2) (layer "F.Cu") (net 3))
 (segment (start 113.15 83.2723) (end 113.15 76.1875) (width 0.2) (layer "B.Cu") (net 6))
 (segment (start 102.2723 94.15) (end 113.15 83.2723) (width 0.2) (layer "B.Cu") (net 6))
 (segment (start 101.905 94.15) (end 102.2723 94.15) (width 0.2) (layer "B.Cu") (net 6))
 (segment (start 117.145 94.722) (end 127.305 104.882) (width 0.2) (layer "B.Cu") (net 2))
 (segment (start 117.145 94.15) (end 117.145 94.722) (width 0.2) (layer "B.Cu") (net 2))
 (segment (start 127.305 118.9175) (end 132.2 123.8125) (width 0.2) (layer "B.Cu") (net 2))
 (segment (start 127.305 104.882) (end 127.305 118.9175) (width 0.2) (layer "B.Cu") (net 2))
 (segment (start 117.145 89.07) (end 115.9509 90.2641) (width 0.2) (layer "F.Cu") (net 13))
 (segment (start 115.9509 92.0504) (end 116.7862 92.8857) (width 0.2) (layer "F.Cu") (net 13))
 (segment (start 115.9509 90.2641) (end 115.9509 92.0504) (width 0.2) (layer "F.Cu") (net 13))
 (segment (start 125.0857 92.8857) (end 132.2 100) (width 0.2) (layer "F.Cu") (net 13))
 (segment (start 116.7862 92.8857) (end 125.0857 92.8857) (width 0.2) (layer "F.Cu") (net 13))
 (segment (start 127.4875 76.1875) (end 132.2 76.1875) (width 0.2) (layer "F.Cu") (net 8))
 (segment (start 117.145 86.53) (end 127.4875 76.1875) (width 0.2) (layer "F.Cu") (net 8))
 (segment (start 114.7996 79.5379) (end 114.7996 68.5554) (width 0.2) (layer "B.Cu") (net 14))
 (segment (start 108.775 130.0511) (end 114.4739 124.3522) (width 0.2) (layer "B.Cu") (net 14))
 (segment (start 114.7996 68.5554) (end 117.145 66.21) (width 0.2) (layer "B.Cu") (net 14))
 (segment (start 114.4739 122.1705) (end 113.8759 121.5725) (width 0.2) (layer "B.Cu") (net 14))
 (segment (start 108.775 133.765) (end 108.775 130.0511) (width 0.2) (layer "B.Cu") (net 14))
 (segment (start 114.4739 124.3522) (end 114.4739 122.1705) (width 0.2) (layer "B.Cu") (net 14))
 (segment (start 113.8759 121.5725) (end 113.8759 103.0903) (width 0.2) (layer "B.Cu") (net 14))
 (segment (start 114.4714 102.4948) (end 114.4714 99.2214) (width 0.2) (layer "B.Cu") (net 14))
 (segment (start 117.145 63.67) (end 117.145 66.21) (width 0.2) (layer "B.Cu") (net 14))
 (segment (start 113.8759 103.0903) (end 114.4714 102.4948) (width 0.2) (layer "B.Cu") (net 14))
 (segment (start 113.9251 98.6751) (end 113.9251 80.4124) (width 0.2) (layer "B.Cu") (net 14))
 (segment (start 114.4714 99.2214) (end 113.9251 98.6751) (width 0.2) (layer "B.Cu") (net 14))
 (segment (start 113.9251 80.4124) (end 114.7996 79.5379) (width 0.2) (layer "B.Cu") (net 14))
 (segment (start 117.145 71.29) (end 115.7635 72.6715) (width 0.2) (layer "F.Cu") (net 16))
 (segment (start 115.7635 72.6715) (end 93.775 72.6715) (width 0.2) (layer "F.Cu") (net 16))
 (via (at 93.775 72.6715) (size 0.6) (drill 0.3) (layers "F.Cu" "B.Cu") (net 16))
 (segment (start 93.775 97.375) (end 93.775 72.6715) (width 0.2) (layer "B.Cu") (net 16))
 (segment (start 93.775 97.375) (end 93.775 102.625) (width 0.2) (layer "B.Cu") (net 16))
 (segment (start 128.575 116.7) (end 128.575 82.4804) (width 0.2) (layer "B.Cu") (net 17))
 (segment (start 128.575 82.4804) (end 119.9246 73.83) (width 0.2) (layer "B.Cu") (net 17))
 (segment (start 119.9246 73.83) (end 117.145 73.83) (width 0.2) (layer "B.Cu") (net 17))
 (segment (start 117.27 109.3233) (end 117.27 102.2586) (width 0.2) (layer "F.Cu") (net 23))
 (segment (start 117.27 102.2586) (end 114.5876 99.5762) (width 0.2) (layer "F.Cu") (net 23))
 (segment (start 114.5876 99.5762) (end 114.5876 98.3826) (width 0.2) (layer "F.Cu") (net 23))
 (segment (start 114.5876 98.3826) (end 105.8882 89.6832) (width 0.2) (layer "F.Cu") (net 23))
 (segment (start 123.495 116.7) (end 123.495 115.5483) (width 0.2) (layer "F.Cu") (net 23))
 (segment (start 123.495 115.5483) (end 117.27 109.3233) (width 0.2) (layer "F.Cu") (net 23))
 (via (at 105.8882 89.6832) (size 0.6) (drill 0.3) (layers "F.Cu" "B.Cu") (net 23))
 (segment (start 105.8882 89.6832) (end 107.2379 88.3335) (width 0.2) (layer "B.Cu") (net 23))
 (segment (start 107.2379 71.5429) (end 101.905 66.21) (width 0.2) (layer "B.Cu") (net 23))
 (segment (start 107.2379 88.3335) (end 107.2379 71.5429) (width 0.2) (layer "B.Cu") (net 23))
 (segment (start 114.9877 91.9927) (end 114.9877 93.7099) (width 0.2) (layer "F.Cu") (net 20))
 (segment (start 118.8122 97.5344) (end 119.815 97.5344) (width 0.2) (layer "F.Cu") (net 20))
 (segment (start 114.9877 93.7099) (end 118.8122 97.5344) (width 0.2) (layer "F.Cu") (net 20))
 (segment (start 101.905 78.91) (end 114.9877 91.9927) (width 0.2) (layer "F.Cu") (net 20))
 (segment (start 131.115 108.8344) (end 131.115 116.7) (width 0.2) (layer "F.Cu") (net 20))
 (segment (start 119.815 97.5344) (end 131.115 108.8344) (width 0.2) (layer "F.Cu") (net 20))
 (segment (start 140.3658 132.4575) (end 107.275 132.4575) (width 0.2) (layer "F.Cu") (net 15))
 (segment (start 146.625 127.1) (end 145.7233 127.1) (width 0.2) (layer "F.Cu") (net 15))
 (segment (start 145.7233 127.1) (end 140.3658 132.4575) (width 0.2) (layer "F.Cu") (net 15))
 (via (at 107.275 132.4575) (size 0.6) (drill 0.3) (layers "F.Cu" "B.Cu") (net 15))
 (segment (start 107.275 133.765) (end 107.275 132.4575) (width 0.2) (layer "B.Cu") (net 15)))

